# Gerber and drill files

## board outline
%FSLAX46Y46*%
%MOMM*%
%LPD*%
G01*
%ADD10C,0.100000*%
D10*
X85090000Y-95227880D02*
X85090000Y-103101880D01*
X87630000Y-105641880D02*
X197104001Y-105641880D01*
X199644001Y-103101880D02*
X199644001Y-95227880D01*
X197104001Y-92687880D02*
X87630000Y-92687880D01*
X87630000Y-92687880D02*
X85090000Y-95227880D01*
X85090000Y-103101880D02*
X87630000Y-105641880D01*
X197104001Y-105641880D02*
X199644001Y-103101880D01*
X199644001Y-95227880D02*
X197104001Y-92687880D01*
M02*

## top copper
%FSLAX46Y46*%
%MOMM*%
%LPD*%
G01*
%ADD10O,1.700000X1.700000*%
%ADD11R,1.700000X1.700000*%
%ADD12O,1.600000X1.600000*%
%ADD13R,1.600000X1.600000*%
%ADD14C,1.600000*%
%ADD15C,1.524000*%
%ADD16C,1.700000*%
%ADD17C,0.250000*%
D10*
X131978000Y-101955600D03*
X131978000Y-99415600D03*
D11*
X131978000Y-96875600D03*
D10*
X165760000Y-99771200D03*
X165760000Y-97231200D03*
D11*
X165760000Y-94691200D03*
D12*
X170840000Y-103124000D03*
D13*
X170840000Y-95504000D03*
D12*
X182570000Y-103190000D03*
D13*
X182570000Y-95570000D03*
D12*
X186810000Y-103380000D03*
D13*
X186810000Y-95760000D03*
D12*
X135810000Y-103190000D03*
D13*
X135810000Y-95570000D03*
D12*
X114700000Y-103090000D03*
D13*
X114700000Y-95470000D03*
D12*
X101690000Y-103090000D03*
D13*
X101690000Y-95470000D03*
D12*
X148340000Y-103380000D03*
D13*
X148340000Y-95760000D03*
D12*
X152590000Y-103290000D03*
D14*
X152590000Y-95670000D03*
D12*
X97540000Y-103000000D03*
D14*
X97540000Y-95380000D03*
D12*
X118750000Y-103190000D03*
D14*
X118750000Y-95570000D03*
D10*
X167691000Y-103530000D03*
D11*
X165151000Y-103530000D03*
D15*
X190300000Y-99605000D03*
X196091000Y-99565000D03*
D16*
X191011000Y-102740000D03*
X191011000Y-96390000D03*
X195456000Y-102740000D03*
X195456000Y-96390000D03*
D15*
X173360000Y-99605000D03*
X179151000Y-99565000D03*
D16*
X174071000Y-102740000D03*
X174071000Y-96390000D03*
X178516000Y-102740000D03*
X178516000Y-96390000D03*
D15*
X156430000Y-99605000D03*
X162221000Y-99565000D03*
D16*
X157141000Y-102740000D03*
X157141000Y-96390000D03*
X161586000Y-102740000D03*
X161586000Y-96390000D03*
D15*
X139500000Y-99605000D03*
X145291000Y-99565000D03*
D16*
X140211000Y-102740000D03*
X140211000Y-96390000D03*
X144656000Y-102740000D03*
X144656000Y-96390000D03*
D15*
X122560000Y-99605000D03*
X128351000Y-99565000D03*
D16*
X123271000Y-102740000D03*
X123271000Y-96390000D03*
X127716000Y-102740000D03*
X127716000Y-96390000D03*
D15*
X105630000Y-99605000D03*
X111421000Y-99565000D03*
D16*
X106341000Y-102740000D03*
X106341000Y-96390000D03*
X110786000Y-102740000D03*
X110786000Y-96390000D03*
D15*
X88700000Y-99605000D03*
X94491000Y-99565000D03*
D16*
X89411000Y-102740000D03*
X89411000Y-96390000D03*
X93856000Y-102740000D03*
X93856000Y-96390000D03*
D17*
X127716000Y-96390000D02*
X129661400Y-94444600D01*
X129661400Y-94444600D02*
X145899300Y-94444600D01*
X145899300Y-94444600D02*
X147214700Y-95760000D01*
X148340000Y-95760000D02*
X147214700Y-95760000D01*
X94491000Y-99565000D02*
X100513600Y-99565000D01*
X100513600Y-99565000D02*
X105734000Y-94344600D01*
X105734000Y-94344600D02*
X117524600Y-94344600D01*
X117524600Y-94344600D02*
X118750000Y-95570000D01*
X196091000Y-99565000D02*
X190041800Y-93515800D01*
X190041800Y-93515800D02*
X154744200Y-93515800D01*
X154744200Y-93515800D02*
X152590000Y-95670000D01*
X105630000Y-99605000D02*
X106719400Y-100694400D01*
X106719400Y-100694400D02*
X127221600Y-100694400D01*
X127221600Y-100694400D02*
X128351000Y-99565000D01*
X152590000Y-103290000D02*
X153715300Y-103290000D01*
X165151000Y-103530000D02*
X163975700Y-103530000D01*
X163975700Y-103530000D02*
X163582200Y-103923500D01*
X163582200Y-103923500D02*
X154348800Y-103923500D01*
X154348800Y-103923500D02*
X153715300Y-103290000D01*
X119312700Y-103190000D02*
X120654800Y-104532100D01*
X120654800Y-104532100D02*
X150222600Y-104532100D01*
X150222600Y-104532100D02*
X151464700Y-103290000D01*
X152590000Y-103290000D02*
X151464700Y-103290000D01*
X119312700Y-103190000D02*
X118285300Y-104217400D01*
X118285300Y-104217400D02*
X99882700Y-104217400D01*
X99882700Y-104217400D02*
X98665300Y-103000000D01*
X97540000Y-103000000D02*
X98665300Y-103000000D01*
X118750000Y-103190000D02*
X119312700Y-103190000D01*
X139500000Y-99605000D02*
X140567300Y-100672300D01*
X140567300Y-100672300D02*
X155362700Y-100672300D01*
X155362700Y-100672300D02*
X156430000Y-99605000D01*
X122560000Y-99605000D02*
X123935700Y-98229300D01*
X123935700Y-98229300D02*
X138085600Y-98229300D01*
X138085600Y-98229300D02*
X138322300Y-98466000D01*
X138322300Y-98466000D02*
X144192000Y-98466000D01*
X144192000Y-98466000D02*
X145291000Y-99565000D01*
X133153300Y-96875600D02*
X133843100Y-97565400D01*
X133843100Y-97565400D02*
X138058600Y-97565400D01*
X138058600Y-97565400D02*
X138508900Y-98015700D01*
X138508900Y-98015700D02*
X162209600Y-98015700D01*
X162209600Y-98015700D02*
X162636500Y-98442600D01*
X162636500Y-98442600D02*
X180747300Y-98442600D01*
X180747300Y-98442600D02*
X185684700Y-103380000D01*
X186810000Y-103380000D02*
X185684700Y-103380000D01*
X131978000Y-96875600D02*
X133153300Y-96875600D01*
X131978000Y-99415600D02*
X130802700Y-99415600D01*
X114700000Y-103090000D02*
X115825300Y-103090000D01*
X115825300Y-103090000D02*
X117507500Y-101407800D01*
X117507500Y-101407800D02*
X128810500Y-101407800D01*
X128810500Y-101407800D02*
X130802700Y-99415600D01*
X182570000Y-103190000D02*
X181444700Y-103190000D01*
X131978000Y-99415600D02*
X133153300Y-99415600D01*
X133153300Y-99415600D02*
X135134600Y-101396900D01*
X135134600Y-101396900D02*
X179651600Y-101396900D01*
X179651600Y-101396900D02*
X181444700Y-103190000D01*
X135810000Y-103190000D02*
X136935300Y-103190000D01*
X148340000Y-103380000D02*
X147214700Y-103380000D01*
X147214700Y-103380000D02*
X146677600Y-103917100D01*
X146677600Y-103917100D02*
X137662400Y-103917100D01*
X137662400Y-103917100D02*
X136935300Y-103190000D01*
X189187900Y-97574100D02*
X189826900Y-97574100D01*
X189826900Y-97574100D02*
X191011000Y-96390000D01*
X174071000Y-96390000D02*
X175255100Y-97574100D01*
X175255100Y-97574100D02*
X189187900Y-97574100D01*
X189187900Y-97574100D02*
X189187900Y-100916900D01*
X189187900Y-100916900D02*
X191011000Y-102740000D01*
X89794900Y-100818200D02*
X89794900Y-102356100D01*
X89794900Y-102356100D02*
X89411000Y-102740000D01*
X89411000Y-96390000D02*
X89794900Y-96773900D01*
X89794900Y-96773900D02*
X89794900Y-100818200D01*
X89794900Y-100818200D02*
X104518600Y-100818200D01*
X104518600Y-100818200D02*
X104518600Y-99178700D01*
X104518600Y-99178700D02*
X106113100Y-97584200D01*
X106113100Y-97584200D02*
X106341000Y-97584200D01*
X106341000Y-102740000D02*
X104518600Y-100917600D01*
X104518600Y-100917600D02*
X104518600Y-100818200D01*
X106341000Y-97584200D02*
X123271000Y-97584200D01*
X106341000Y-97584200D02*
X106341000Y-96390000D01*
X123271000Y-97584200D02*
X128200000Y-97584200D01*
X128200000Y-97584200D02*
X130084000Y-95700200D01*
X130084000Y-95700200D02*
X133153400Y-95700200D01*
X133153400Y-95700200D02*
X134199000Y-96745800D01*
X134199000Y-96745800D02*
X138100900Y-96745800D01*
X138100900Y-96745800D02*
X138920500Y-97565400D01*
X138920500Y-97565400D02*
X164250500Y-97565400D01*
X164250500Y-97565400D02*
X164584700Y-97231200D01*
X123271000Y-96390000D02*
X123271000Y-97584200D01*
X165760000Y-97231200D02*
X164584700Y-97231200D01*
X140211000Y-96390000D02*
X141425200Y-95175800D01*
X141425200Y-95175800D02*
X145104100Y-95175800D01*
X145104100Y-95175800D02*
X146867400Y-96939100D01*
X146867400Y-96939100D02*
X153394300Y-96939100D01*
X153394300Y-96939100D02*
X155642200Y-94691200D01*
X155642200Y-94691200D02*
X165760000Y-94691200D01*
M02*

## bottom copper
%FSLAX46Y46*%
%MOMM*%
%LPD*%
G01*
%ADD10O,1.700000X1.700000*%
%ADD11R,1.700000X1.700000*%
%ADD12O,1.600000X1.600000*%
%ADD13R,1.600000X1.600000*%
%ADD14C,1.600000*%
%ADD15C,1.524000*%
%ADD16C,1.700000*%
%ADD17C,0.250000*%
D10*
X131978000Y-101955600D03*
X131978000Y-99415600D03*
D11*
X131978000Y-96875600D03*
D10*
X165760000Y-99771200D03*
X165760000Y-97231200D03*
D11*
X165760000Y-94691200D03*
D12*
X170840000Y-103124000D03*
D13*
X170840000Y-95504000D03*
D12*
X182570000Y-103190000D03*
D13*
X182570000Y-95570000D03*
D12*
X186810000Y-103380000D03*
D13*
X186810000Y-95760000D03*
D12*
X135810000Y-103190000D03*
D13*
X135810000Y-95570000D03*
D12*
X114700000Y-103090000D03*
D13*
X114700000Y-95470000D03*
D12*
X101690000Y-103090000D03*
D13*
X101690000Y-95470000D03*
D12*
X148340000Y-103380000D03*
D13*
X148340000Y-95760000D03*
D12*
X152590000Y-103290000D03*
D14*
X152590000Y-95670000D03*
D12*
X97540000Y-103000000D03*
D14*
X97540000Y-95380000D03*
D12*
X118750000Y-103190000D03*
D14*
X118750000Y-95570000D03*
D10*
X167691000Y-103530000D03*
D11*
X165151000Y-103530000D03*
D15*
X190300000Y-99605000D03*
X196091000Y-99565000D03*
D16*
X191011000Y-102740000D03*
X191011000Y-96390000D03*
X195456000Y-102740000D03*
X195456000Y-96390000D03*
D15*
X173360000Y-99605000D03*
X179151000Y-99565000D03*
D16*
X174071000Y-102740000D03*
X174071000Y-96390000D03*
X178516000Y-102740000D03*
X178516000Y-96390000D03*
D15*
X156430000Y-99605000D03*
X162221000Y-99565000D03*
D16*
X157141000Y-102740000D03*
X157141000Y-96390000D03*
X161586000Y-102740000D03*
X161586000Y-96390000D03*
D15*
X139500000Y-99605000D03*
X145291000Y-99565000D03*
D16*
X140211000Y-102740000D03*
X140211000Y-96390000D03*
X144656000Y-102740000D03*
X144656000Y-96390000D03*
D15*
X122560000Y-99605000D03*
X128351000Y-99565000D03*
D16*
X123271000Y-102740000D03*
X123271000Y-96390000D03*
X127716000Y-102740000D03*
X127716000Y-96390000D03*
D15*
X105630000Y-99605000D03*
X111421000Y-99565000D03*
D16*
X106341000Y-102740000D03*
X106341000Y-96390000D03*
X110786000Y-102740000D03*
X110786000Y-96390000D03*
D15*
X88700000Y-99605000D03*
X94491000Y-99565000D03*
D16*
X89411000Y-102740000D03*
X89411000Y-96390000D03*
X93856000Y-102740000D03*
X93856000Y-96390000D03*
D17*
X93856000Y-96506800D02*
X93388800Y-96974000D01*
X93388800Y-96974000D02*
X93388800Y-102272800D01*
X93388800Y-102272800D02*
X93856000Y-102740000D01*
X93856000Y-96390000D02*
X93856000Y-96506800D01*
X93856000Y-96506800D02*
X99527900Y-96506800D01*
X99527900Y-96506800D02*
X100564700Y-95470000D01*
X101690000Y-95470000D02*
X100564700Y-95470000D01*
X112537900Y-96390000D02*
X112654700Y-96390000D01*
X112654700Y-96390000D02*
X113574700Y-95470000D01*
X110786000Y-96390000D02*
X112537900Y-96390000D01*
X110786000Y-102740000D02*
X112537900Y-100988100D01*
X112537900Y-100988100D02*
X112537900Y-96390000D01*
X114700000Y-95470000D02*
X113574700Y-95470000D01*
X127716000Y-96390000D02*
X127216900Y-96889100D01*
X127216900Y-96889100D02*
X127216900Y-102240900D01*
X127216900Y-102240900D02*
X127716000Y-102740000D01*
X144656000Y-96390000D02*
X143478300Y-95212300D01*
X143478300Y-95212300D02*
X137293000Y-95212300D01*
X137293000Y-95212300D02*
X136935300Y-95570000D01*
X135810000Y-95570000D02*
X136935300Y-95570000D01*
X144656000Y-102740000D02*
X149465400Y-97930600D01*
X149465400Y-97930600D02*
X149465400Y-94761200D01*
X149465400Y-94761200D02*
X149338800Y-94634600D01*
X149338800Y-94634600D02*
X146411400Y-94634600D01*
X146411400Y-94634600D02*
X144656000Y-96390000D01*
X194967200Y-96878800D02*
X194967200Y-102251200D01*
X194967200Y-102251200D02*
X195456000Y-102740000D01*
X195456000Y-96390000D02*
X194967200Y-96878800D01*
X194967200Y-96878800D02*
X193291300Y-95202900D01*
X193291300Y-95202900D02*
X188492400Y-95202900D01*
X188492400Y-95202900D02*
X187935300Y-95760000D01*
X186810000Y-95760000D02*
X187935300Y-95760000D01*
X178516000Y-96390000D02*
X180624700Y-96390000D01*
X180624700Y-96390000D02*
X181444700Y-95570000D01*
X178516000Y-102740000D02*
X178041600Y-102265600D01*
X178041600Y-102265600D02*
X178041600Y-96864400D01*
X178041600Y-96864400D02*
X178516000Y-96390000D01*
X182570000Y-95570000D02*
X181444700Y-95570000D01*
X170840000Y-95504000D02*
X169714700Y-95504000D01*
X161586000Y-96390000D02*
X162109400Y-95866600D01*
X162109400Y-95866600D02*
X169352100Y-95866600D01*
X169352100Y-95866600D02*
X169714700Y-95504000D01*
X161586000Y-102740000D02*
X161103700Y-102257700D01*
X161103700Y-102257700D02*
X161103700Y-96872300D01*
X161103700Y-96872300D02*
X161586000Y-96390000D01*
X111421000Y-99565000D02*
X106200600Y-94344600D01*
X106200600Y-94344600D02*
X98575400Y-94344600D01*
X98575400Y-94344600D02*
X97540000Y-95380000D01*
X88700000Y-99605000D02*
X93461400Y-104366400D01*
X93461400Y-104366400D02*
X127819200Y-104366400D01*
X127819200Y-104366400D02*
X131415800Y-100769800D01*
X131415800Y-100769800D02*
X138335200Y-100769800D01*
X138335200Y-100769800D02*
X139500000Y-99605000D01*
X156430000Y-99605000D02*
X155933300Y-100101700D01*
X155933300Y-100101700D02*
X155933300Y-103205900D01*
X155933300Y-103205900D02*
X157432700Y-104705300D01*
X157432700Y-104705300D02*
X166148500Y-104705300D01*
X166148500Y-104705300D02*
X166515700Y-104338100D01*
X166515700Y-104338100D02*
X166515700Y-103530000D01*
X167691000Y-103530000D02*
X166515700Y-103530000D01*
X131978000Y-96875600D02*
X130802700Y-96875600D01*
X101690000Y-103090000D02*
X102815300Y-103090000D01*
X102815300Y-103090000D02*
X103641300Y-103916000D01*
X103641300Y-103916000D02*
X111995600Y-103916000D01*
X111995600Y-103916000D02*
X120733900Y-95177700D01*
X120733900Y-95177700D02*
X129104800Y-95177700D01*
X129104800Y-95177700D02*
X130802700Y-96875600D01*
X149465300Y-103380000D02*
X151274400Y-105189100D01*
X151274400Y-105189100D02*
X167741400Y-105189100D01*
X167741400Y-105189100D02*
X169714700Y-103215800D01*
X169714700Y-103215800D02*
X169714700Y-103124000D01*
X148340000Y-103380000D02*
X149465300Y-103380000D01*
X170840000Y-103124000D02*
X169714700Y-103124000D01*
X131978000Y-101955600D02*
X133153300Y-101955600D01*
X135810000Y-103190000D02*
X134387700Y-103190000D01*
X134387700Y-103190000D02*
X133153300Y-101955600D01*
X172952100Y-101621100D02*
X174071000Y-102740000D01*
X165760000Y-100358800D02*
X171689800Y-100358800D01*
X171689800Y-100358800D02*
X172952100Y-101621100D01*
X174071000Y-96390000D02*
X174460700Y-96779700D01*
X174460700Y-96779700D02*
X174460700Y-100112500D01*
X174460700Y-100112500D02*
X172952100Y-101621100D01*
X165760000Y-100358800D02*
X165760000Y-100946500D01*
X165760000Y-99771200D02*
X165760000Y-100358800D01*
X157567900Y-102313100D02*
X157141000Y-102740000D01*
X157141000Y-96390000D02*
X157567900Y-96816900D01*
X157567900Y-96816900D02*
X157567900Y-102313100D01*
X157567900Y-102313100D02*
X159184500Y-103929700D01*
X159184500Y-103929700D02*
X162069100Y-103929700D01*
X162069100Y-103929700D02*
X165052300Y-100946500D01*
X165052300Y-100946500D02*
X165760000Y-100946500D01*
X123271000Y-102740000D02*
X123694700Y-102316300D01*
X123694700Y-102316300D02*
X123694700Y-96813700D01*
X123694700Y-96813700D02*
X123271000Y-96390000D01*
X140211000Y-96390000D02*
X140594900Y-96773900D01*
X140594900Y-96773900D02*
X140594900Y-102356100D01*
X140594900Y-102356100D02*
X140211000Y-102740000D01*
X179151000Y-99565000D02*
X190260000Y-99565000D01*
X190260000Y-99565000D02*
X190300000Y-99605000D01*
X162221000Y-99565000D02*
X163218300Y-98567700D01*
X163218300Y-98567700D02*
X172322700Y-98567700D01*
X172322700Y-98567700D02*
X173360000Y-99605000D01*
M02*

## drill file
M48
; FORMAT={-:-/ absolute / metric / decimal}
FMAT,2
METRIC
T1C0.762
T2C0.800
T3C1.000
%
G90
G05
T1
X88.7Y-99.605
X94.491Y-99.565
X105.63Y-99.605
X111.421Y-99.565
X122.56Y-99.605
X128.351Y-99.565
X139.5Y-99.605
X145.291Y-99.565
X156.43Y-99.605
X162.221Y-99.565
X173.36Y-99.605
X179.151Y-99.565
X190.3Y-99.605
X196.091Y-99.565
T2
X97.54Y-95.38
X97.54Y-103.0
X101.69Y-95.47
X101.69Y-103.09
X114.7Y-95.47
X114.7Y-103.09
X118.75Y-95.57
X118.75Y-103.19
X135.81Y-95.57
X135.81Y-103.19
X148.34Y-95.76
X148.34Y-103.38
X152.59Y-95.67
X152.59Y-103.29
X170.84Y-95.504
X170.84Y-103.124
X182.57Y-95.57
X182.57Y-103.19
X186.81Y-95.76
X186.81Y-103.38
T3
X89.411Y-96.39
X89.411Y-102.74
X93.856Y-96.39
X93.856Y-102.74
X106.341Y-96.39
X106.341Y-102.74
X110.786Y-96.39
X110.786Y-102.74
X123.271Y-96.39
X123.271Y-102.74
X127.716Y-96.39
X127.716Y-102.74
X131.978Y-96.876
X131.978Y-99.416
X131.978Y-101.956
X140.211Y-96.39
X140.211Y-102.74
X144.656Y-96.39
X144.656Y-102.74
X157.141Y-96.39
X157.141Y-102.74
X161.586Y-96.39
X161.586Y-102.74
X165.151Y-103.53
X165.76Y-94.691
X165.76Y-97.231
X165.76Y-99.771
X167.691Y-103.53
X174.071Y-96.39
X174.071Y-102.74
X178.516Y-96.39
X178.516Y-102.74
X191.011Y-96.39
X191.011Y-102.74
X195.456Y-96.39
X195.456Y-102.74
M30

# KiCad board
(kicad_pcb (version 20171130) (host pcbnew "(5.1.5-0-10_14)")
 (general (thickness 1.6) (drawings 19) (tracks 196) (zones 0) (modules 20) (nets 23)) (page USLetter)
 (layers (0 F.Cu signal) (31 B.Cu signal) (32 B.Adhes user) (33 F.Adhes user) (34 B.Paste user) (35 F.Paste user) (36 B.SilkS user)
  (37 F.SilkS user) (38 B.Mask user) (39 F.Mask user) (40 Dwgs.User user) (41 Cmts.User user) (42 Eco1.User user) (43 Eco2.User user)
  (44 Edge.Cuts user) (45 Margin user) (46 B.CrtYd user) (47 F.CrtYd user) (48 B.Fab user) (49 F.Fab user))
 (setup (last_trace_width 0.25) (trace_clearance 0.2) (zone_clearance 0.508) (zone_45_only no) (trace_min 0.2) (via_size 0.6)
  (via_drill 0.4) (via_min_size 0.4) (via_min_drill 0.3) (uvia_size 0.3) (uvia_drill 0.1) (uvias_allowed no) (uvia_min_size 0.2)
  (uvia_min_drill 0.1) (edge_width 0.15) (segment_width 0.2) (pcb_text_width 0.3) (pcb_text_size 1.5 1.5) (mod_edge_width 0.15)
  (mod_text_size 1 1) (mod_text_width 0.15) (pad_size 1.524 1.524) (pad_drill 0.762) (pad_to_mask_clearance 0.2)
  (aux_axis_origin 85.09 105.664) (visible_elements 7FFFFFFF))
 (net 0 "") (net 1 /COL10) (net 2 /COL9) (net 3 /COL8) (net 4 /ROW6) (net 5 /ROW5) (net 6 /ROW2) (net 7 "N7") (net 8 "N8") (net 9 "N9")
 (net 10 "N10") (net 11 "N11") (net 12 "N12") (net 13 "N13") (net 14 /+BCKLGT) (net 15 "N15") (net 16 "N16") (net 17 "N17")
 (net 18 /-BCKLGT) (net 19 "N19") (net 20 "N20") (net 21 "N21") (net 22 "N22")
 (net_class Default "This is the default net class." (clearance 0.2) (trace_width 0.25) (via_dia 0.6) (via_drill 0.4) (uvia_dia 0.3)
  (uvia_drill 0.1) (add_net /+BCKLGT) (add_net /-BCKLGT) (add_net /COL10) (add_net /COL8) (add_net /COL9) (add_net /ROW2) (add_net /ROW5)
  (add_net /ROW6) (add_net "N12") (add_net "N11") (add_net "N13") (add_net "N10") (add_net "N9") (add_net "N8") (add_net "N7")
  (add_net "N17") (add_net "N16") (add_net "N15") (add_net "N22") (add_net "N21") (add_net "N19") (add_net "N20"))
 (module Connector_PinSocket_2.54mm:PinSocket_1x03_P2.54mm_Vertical (layer F.Cu) (at 131.978 96.8756)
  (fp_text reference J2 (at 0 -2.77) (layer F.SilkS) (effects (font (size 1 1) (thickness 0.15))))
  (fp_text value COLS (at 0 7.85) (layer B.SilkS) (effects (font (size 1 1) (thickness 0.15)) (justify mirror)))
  (pad 3 thru_hole oval (at 0 5.08) (size 1.7 1.7) (drill 1) (layers *.Cu *.Mask) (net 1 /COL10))
  (pad 2 thru_hole oval (at 0 2.54) (size 1.7 1.7) (drill 1) (layers *.Cu *.Mask) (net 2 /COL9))
  (pad 1 thru_hole rect (at 0 0) (size 1.7 1.7) (drill 1) (layers *.Cu *.Mask) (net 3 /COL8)))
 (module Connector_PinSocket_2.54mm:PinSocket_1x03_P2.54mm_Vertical (layer F.Cu) (at 165.76 94.6912)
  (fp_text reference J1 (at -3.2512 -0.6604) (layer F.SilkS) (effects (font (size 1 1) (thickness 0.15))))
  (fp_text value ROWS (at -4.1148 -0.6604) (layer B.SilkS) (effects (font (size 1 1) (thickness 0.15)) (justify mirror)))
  (pad 3 thru_hole oval (at 0 5.08) (size 1.7 1.7) (drill 1) (layers *.Cu *.Mask) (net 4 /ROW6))
  (pad 2 thru_hole oval (at 0 2.54) (size 1.7 1.7) (drill 1) (layers *.Cu *.Mask) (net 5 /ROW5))
  (pad 1 thru_hole rect (at 0 0) (size 1.7 1.7) (drill 1) (layers *.Cu *.Mask) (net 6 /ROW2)))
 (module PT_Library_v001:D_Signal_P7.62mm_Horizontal (layer F.Cu) (at 170.84 95.504 270)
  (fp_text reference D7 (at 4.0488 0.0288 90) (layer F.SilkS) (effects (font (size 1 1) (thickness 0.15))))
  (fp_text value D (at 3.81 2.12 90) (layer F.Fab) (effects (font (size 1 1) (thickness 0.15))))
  (pad 2 thru_hole oval (at 7.62 0 270) (size 1.6 1.6) (drill 0.8) (layers *.Cu *.Mask) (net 1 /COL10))
  (pad 1 thru_hole rect (at 0 0 270) (size 1.6 1.6) (drill 0.8) (layers *.Cu *.Mask) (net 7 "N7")))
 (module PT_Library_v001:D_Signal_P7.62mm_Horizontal (layer F.Cu) (at 182.57 95.57 270)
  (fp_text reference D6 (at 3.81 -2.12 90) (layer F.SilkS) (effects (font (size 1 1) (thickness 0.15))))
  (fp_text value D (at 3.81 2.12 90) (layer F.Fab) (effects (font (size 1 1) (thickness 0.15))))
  (pad 2 thru_hole oval (at 7.62 0 270) (size 1.6 1.6) (drill 0.8) (layers *.Cu *.Mask) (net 2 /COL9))
  (pad 1 thru_hole rect (at 0 0 270) (size 1.6 1.6) (drill 0.8) (layers *.Cu *.Mask) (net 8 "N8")))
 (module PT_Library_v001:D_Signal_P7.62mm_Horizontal (layer F.Cu) (at 186.81 95.76 270)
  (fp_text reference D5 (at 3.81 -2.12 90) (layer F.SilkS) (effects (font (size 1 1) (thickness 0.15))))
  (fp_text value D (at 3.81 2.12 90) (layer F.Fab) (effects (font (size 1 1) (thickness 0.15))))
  (pad 2 thru_hole oval (at 7.62 0 270) (size 1.6 1.6) (drill 0.8) (layers *.Cu *.Mask) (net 3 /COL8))
  (pad 1 thru_hole rect (at 0 0 270) (size 1.6 1.6) (drill 0.8) (layers *.Cu *.Mask) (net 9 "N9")))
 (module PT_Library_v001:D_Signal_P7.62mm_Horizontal (layer F.Cu) (at 135.81 95.57 270)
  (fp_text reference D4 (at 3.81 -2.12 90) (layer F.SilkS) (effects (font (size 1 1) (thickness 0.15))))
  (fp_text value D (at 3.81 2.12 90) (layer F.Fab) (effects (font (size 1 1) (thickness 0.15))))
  (pad 2 thru_hole oval (at 7.62 0 270) (size 1.6 1.6) (drill 0.8) (layers *.Cu *.Mask) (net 1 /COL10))
  (pad 1 thru_hole rect (at 0 0 270) (size 1.6 1.6) (drill 0.8) (layers *.Cu *.Mask) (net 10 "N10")))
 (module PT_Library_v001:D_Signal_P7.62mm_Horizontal (layer F.Cu) (at 114.7 95.47 270)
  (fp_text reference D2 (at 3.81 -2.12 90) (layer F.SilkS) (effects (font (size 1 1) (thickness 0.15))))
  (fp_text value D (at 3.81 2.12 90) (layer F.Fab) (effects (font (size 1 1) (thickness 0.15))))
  (pad 2 thru_hole oval (at 7.62 0 270) (size 1.6 1.6) (drill 0.8) (layers *.Cu *.Mask) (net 2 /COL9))
  (pad 1 thru_hole rect (at 0 0 270) (size 1.6 1.6) (drill 0.8) (layers *.Cu *.Mask) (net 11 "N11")))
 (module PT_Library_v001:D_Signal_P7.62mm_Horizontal (layer F.Cu) (at 101.69 95.47 270)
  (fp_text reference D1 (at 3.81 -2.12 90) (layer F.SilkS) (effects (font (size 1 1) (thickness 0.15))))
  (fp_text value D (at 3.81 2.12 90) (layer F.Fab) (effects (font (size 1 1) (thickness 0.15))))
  (pad 2 thru_hole oval (at 7.62 0 270) (size 1.6 1.6) (drill 0.8) (layers *.Cu *.Mask) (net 3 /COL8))
  (pad 1 thru_hole rect (at 0 0 270) (size 1.6 1.6) (drill 0.8) (layers *.Cu *.Mask) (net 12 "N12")))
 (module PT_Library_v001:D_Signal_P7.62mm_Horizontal (layer F.Cu) (at 148.34 95.76 270)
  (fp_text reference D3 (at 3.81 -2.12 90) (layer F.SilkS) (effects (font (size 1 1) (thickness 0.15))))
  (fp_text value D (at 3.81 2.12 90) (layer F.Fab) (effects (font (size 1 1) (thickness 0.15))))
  (pad 2 thru_hole oval (at 7.62 0 270) (size 1.6 1.6) (drill 0.8) (layers *.Cu *.Mask) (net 1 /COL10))
  (pad 1 thru_hole rect (at 0 0 270) (size 1.6 1.6) (drill 0.8) (layers *.Cu *.Mask) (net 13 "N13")))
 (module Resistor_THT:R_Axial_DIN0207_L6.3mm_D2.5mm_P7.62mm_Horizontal (layer F.Cu) (at 152.59 95.67 270)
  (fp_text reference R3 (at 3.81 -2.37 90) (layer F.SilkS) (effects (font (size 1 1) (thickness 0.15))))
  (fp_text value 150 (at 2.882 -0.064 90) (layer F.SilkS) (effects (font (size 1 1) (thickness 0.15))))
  (pad 2 thru_hole oval (at 7.62 0 270) (size 1.6 1.6) (drill 0.8) (layers *.Cu *.Mask) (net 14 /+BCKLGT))
  (pad 1 thru_hole circle (at 0 0 270) (size 1.6 1.6) (drill 0.8) (layers *.Cu *.Mask) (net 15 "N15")))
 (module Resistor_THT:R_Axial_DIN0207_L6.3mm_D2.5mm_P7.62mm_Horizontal (layer F.Cu) (at 97.54 95.38 270)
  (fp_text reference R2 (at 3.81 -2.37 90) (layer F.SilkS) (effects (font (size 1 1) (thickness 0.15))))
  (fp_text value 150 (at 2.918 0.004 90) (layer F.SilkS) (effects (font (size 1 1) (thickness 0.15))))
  (pad 2 thru_hole oval (at 7.62 0 270) (size 1.6 1.6) (drill 0.8) (layers *.Cu *.Mask) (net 14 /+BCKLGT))
  (pad 1 thru_hole circle (at 0 0 270) (size 1.6 1.6) (drill 0.8) (layers *.Cu *.Mask) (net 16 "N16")))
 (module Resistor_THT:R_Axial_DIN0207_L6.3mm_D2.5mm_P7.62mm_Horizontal (layer F.Cu) (at 118.75 95.57 270)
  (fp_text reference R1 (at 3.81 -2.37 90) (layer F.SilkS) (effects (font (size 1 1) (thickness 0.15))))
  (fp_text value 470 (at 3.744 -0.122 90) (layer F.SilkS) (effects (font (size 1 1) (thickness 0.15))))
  (pad 2 thru_hole oval (at 7.62 0 270) (size 1.6 1.6) (drill 0.8) (layers *.Cu *.Mask) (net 14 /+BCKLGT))
  (pad 1 thru_hole circle (at 0 0 270) (size 1.6 1.6) (drill 0.8) (layers *.Cu *.Mask) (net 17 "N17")))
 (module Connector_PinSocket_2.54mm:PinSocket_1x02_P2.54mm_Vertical (layer B.Cu) (at 165.151 103.53 270)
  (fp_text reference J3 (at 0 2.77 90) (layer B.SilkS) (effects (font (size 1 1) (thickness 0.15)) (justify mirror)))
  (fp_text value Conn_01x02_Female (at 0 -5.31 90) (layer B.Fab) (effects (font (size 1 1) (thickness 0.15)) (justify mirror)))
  (pad 2 thru_hole oval (at 0 -2.54 270) (size 1.7 1.7) (drill 1) (layers *.Cu *.Mask) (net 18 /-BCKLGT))
  (pad 1 thru_hole rect (at 0 0 270) (size 1.7 1.7) (drill 1) (layers *.Cu *.Mask) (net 14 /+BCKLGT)))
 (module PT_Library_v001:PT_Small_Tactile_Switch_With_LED (layer F.Cu) (at 193.17 99.565 270)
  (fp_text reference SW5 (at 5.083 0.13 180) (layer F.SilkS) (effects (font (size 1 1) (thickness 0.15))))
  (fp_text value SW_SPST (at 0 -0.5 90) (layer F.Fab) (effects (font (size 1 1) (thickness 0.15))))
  (pad 6 thru_hole circle (at 0.04 2.87 270) (size 1.524 1.524) (drill 0.762) (layers *.Cu *.Mask) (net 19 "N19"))
  (pad 5 thru_hole circle (at 0 -2.921 270) (size 1.524 1.524) (drill 0.762) (layers *.Cu *.Mask) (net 15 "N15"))
  (pad 4 thru_hole circle (at 3.175 2.159 270) (size 1.7 1.7) (drill 1) (layers *.Cu *.Mask) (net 4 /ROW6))
  (pad 3 thru_hole circle (at -3.175 2.159 270) (size 1.7 1.7) (drill 1) (layers *.Cu *.Mask) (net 4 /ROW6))
  (pad 2 thru_hole circle (at 3.175 -2.286 270) (size 1.7 1.7) (drill 1) (layers *.Cu *.Mask) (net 9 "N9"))
  (pad 1 thru_hole circle (at -3.175 -2.286 270) (size 1.7 1.7) (drill 1) (layers *.Cu *.Mask) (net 9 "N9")))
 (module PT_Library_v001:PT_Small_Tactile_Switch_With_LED (layer F.Cu) (at 176.23 99.565 270)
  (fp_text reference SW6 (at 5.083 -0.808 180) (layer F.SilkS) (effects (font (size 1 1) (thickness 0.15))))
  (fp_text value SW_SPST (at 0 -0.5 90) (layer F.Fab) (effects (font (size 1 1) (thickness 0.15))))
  (pad 6 thru_hole circle (at 0.04 2.87 270) (size 1.524 1.524) (drill 0.762) (layers *.Cu *.Mask) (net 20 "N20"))
  (pad 5 thru_hole circle (at 0 -2.921 270) (size 1.524 1.524) (drill 0.762) (layers *.Cu *.Mask) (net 19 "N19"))
  (pad 4 thru_hole circle (at 3.175 2.159 270) (size 1.7 1.7) (drill 1) (layers *.Cu *.Mask) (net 4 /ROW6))
  (pad 3 thru_hole circle (at -3.175 2.159 270) (size 1.7 1.7) (drill 1) (layers *.Cu *.Mask) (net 4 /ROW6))
  (pad 2 thru_hole circle (at 3.175 -2.286 270) (size 1.7 1.7) (drill 1) (layers *.Cu *.Mask) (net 8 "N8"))
  (pad 1 thru_hole circle (at -3.175 -2.286 270) (size 1.7 1.7) (drill 1) (layers *.Cu *.Mask) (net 8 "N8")))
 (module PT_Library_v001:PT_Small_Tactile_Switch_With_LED (layer F.Cu) (at 159.3 99.565 270)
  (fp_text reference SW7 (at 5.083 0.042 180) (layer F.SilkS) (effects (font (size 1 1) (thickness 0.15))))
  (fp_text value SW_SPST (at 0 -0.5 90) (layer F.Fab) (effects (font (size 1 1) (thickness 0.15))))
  (pad 6 thru_hole circle (at 0.04 2.87 270) (size 1.524 1.524) (drill 0.762) (layers *.Cu *.Mask) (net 18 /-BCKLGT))
  (pad 5 thru_hole circle (at 0 -2.921 270) (size 1.524 1.524) (drill 0.762) (layers *.Cu *.Mask) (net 20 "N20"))
  (pad 4 thru_hole circle (at 3.175 2.159 270) (size 1.7 1.7) (drill 1) (layers *.Cu *.Mask) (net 4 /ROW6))
  (pad 3 thru_hole circle (at -3.175 2.159 270) (size 1.7 1.7) (drill 1) (layers *.Cu *.Mask) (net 4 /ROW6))
  (pad 2 thru_hole circle (at 3.175 -2.286 270) (size 1.7 1.7) (drill 1) (layers *.Cu *.Mask) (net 7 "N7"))
  (pad 1 thru_hole circle (at -3.175 -2.286 270) (size 1.7 1.7) (drill 1) (layers *.Cu *.Mask) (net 7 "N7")))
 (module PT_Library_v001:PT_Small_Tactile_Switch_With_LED (layer F.Cu) (at 142.37 99.565 270)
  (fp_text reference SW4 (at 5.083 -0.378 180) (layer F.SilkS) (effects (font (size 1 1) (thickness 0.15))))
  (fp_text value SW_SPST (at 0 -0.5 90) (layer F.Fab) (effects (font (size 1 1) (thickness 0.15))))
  (pad 6 thru_hole circle (at 0.04 2.87 270) (size 1.524 1.524) (drill 0.762) (layers *.Cu *.Mask) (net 18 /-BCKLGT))
  (pad 5 thru_hole circle (at 0 -2.921 270) (size 1.524 1.524) (drill 0.762) (layers *.Cu *.Mask) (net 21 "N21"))
  (pad 4 thru_hole circle (at 3.175 2.159 270) (size 1.7 1.7) (drill 1) (layers *.Cu *.Mask) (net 6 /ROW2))
  (pad 3 thru_hole circle (at -3.175 2.159 270) (size 1.7 1.7) (drill 1) (layers *.Cu *.Mask) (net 6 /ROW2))
  (pad 2 thru_hole circle (at 3.175 -2.286 270) (size 1.7 1.7) (drill 1) (layers *.Cu *.Mask) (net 10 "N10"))
  (pad 1 thru_hole circle (at -3.175 -2.286 270) (size 1.7 1.7) (drill 1) (layers *.Cu *.Mask) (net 10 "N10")))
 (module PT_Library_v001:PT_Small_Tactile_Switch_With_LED (layer F.Cu) (at 125.43 99.565 270)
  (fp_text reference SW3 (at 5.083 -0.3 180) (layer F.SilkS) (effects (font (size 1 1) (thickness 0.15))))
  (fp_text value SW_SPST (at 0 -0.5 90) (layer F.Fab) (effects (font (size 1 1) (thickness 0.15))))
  (pad 6 thru_hole circle (at 0.04 2.87 270) (size 1.524 1.524) (drill 0.762) (layers *.Cu *.Mask) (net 21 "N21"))
  (pad 5 thru_hole circle (at 0 -2.921 270) (size 1.524 1.524) (drill 0.762) (layers *.Cu *.Mask) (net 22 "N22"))
  (pad 4 thru_hole circle (at 3.175 2.159 270) (size 1.7 1.7) (drill 1) (layers *.Cu *.Mask) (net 5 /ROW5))
  (pad 3 thru_hole circle (at -3.175 2.159 270) (size 1.7 1.7) (drill 1) (layers *.Cu *.Mask) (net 5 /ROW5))
  (pad 2 thru_hole circle (at 3.175 -2.286 270) (size 1.7 1.7) (drill 1) (layers *.Cu *.Mask) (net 13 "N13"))
  (pad 1 thru_hole circle (at -3.175 -2.286 270) (size 1.7 1.7) (drill 1) (layers *.Cu *.Mask) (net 13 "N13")))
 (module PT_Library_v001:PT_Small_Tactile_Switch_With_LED (layer F.Cu) (at 108.5 99.565 270)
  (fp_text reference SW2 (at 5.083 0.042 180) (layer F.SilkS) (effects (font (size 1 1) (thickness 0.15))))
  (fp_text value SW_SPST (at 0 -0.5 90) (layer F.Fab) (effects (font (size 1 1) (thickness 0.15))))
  (pad 6 thru_hole circle (at 0.04 2.87 270) (size 1.524 1.524) (drill 0.762) (layers *.Cu *.Mask) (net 22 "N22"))
  (pad 5 thru_hole circle (at 0 -2.921 270) (size 1.524 1.524) (drill 0.762) (layers *.Cu *.Mask) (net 16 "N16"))
  (pad 4 thru_hole circle (at 3.175 2.159 270) (size 1.7 1.7) (drill 1) (layers *.Cu *.Mask) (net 5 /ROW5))
  (pad 3 thru_hole circle (at -3.175 2.159 270) (size 1.7 1.7) (drill 1) (layers *.Cu *.Mask) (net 5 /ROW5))
  (pad 2 thru_hole circle (at 3.175 -2.286 270) (size 1.7 1.7) (drill 1) (layers *.Cu *.Mask) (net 11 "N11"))
  (pad 1 thru_hole circle (at -3.175 -2.286 270) (size 1.7 1.7) (drill 1) (layers *.Cu *.Mask) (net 11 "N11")))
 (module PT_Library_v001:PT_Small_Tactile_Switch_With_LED (layer F.Cu) (at 91.57 99.565 270)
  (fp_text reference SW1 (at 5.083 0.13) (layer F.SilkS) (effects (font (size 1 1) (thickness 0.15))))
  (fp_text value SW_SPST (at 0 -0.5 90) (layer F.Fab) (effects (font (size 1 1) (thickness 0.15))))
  (pad 6 thru_hole circle (at 0.04 2.87 270) (size 1.524 1.524) (drill 0.762) (layers *.Cu *.Mask) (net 18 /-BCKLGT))
  (pad 5 thru_hole circle (at 0 -2.921 270) (size 1.524 1.524) (drill 0.762) (layers *.Cu *.Mask) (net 17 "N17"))
  (pad 4 thru_hole circle (at 3.175 2.159 270) (size 1.7 1.7) (drill 1) (layers *.Cu *.Mask) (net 5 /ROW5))
  (pad 3 thru_hole circle (at -3.175 2.159 270) (size 1.7 1.7) (drill 1) (layers *.Cu *.Mask) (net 5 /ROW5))
  (pad 2 thru_hole circle (at 3.175 -2.286 270) (size 1.7 1.7) (drill 1) (layers *.Cu *.Mask) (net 12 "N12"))
  (pad 1 thru_hole circle (at -3.175 -2.286 270) (size 1.7 1.7) (drill 1) (layers *.Cu *.Mask) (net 12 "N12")))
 (gr_line (start 85.09 95.22788) (end 85.09 103.10188) (layer Edge.Cuts) (width 0.1))
 (gr_line (start 87.63 105.64188) (end 197.104001 105.64188) (layer Edge.Cuts) (width 0.1))
 (gr_line (start 199.644001 103.10188) (end 199.644001 95.22788) (layer Edge.Cuts) (width 0.1))
 (gr_line (start 197.104001 92.68788) (end 87.63 92.68788) (layer Edge.Cuts) (width 0.1))
 (gr_line (start 87.63 92.68788) (end 85.09 95.22788) (layer Edge.Cuts) (width 0.1))
 (gr_line (start 85.09 103.10188) (end 87.63 105.64188) (layer Edge.Cuts) (width 0.1))
 (gr_line (start 197.104001 105.64188) (end 199.644001 103.10188) (layer Edge.Cuts) (width 0.1))
 (gr_line (start 199.644001 95.22788) (end 197.104001 92.68788) (layer Edge.Cuts) (width 0.1))
 (segment (start 93.856 96.5068) (end 93.3888 96.974) (width 0.25) (layer B.Cu) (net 12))
 (segment (start 93.3888 96.974) (end 93.3888 102.2728) (width 0.25) (layer B.Cu) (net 12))
 (segment (start 93.3888 102.2728) (end 93.856 102.74) (width 0.25) (layer B.Cu) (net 12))
 (segment (start 93.856 96.39) (end 93.856 96.5068) (width 0.25) (layer B.Cu) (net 12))
 (segment (start 93.856 96.5068) (end 99.5279 96.5068) (width 0.25) (layer B.Cu) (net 12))
 (segment (start 99.5279 96.5068) (end 100.5647 95.47) (width 0.25) (layer B.Cu) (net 12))
 (segment (start 101.69 95.47) (end 100.5647 95.47) (width 0.25) (layer B.Cu) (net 12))
 (segment (start 112.5379 96.39) (end 112.6547 96.39) (width 0.25) (layer B.Cu) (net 11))
 (segment (start 112.6547 96.39) (end 113.5747 95.47) (width 0.25) (layer B.Cu) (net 11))
 (segment (start 110.786 96.39) (end 112.5379 96.39) (width 0.25) (layer B.Cu) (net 11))
 (segment (start 110.786 102.74) (end 112.5379 100.9881) (width 0.25) (layer B.Cu) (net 11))
 (segment (start 112.5379 100.9881) (end 112.5379 96.39) (width 0.25) (layer B.Cu) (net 11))
 (segment (start 114.7 95.47) (end 113.5747 95.47) (width 0.25) (layer B.Cu) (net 11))
 (segment (start 127.716 96.39) (end 127.2169 96.8891) (width 0.25) (layer B.Cu) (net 13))
 (segment (start 127.2169 96.8891) (end 127.2169 102.2409) (width 0.25) (layer B.Cu) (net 13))
 (segment (start 127.2169 102.2409) (end 127.716 102.74) (width 0.25) (layer B.Cu) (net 13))
 (segment (start 127.716 96.39) (end 129.6614 94.4446) (width 0.25) (layer F.Cu) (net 13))
 (segment (start 129.6614 94.4446) (end 145.8993 94.4446) (width 0.25) (layer F.Cu) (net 13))
 (segment (start 145.8993 94.4446) (end 147.2147 95.76) (width 0.25) (layer F.Cu) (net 13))
 (segment (start 148.34 95.76) (end 147.2147 95.76) (width 0.25) (layer F.Cu) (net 13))
 (segment (start 144.656 96.39) (end 143.4783 95.2123) (width 0.25) (layer B.Cu) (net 10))
 (segment (start 143.4783 95.2123) (end 137.293 95.2123) (width 0.25) (layer B.Cu) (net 10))
 (segment (start 137.293 95.2123) (end 136.9353 95.57) (width 0.25) (layer B.Cu) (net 10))
 (segment (start 135.81 95.57) (end 136.9353 95.57) (width 0.25) (layer B.Cu) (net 10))
 (segment (start 144.656 102.74) (end 149.4654 97.9306) (width 0.25) (layer B.Cu) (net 10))
 (segment (start 149.4654 97.9306) (end 149.4654 94.7612) (width 0.25) (layer B.Cu) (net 10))
 (segment (start 149.4654 94.7612) (end 149.3388 94.6346) (width 0.25) (layer B.Cu) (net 10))
 (segment (start 149.3388 94.6346) (end 146.4114 94.6346) (width 0.25) (layer B.Cu) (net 10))
 (segment (start 146.4114 94.6346) (end 144.656 96.39) (width 0.25) (layer B.Cu) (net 10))
 (segment (start 194.9672 96.8788) (end 194.9672 102.2512) (width 0.25) (layer B.Cu) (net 9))
 (segment (start 194.9672 102.2512) (end 195.456 102.74) (width 0.25) (layer B.Cu) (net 9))
 (segment (start 195.456 96.39) (end 194.9672 96.8788) (width 0.25) (layer B.Cu) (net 9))
 (segment (start 194.9672 96.8788) (end 193.2913 95.2029) (width 0.25) (layer B.Cu) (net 9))
 (segment (start 193.2913 95.2029) (end 188.4924 95.2029) (width 0.25) (layer B.Cu) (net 9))
 (segment (start 188.4924 95.2029) (end 187.9353 95.76) (width 0.25) (layer B.Cu) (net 9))
 (segment (start 186.81 95.76) (end 187.9353 95.76) (width 0.25) (layer B.Cu) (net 9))
 (segment (start 178.516 96.39) (end 180.6247 96.39) (width 0.25) (layer B.Cu) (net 8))
 (segment (start 180.6247 96.39) (end 181.4447 95.57) (width 0.25) (layer B.Cu) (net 8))
 (segment (start 178.516 102.74) (end 178.0416 102.2656) (width 0.25) (layer B.Cu) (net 8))
 (segment (start 178.0416 102.2656) (end 178.0416 96.8644) (width 0.25) (layer B.Cu) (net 8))
 (segment (start 178.0416 96.8644) (end 178.516 96.39) (width 0.25) (layer B.Cu) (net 8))
 (segment (start 182.57 95.57) (end 181.4447 95.57) (width 0.25) (layer B.Cu) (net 8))
 (segment (start 170.84 95.504) (end 169.7147 95.504) (width 0.25) (layer B.Cu) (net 7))
 (segment (start 161.586 96.39) (end 162.1094 95.8666) (width 0.25) (layer B.Cu) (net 7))
 (segment (start 162.1094 95.8666) (end 169.3521 95.8666) (width 0.25) (layer B.Cu) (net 7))
 (segment (start 169.3521 95.8666) (end 169.7147 95.504) (width 0.25) (layer B.Cu) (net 7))
 (segment (start 161.586 102.74) (end 161.1037 102.2577) (width 0.25) (layer B.Cu) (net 7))
 (segment (start 161.1037 102.2577) (end 161.1037 96.8723) (width 0.25) (layer B.Cu) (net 7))
 (segment (start 161.1037 96.8723) (end 161.586 96.39) (width 0.25) (layer B.Cu) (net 7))
 (segment (start 94.491 99.565) (end 100.5136 99.565) (width 0.25) (layer F.Cu) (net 17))
 (segment (start 100.5136 99.565) (end 105.734 94.3446) (width 0.25) (layer F.Cu) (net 17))
 (segment (start 105.734 94.3446) (end 117.5246 94.3446) (width 0.25) (layer F.Cu) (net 17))
 (segment (start 117.5246 94.3446) (end 118.75 95.57) (width 0.25) (layer F.Cu) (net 17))
 (segment (start 111.421 99.565) (end 106.2006 94.3446) (width 0.25) (layer B.Cu) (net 16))
 (segment (start 106.2006 94.3446) (end 98.5754 94.3446) (width 0.25) (layer B.Cu) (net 16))
 (segment (start 98.5754 94.3446) (end 97.54 95.38) (width 0.25) (layer B.Cu) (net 16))
 (segment (start 196.091 99.565) (end 190.0418 93.5158) (width 0.25) (layer F.Cu) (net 15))
 (segment (start 190.0418 93.5158) (end 154.7442 93.5158) (width 0.25) (layer F.Cu) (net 15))
 (segment (start 154.7442 93.5158) (end 152.59 95.67) (width 0.25) (layer F.Cu) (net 15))
 (segment (start 105.63 99.605) (end 106.7194 100.6944) (width 0.25) (layer F.Cu) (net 22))
 (segment (start 106.7194 100.6944) (end 127.2216 100.6944) (width 0.25) (layer F.Cu) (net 22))
 (segment (start 127.2216 100.6944) (end 128.351 99.565) (width 0.25) (layer F.Cu) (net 22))
 (segment (start 152.59 103.29) (end 153.7153 103.29) (width 0.25) (layer F.Cu) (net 14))
 (segment (start 165.151 103.53) (end 163.9757 103.53) (width 0.25) (layer F.Cu) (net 14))
 (segment (start 163.9757 103.53) (end 163.5822 103.9235) (width 0.25) (layer F.Cu) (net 14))
 (segment (start 163.5822 103.9235) (end 154.3488 103.9235) (width 0.25) (layer F.Cu) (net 14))
 (segment (start 154.3488 103.9235) (end 153.7153 103.29) (width 0.25) (layer F.Cu) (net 14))
 (segment (start 119.3127 103.19) (end 120.6548 104.5321) (width 0.25) (layer F.Cu) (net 14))
 (segment (start 120.6548 104.5321) (end 150.2226 104.5321) (width 0.25) (layer F.Cu) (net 14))
 (segment (start 150.2226 104.5321) (end 151.4647 103.29) (width 0.25) (layer F.Cu) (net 14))
 (segment (start 152.59 103.29) (end 151.4647 103.29) (width 0.25) (layer F.Cu) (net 14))
 (segment (start 119.3127 103.19) (end 118.2853 104.2174) (width 0.25) (layer F.Cu) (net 14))
 (segment (start 118.2853 104.2174) (end 99.8827 104.2174) (width 0.25) (layer F.Cu) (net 14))
 (segment (start 99.8827 104.2174) (end 98.6653 103) (width 0.25) (layer F.Cu) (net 14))
 (segment (start 97.54 103) (end 98.6653 103) (width 0.25) (layer F.Cu) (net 14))
 (segment (start 118.75 103.19) (end 119.3127 103.19) (width 0.25) (layer F.Cu) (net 14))
 (segment (start 88.7 99.605) (end 93.4614 104.3664) (width 0.25) (layer B.Cu) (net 18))
 (segment (start 93.4614 104.3664) (end 127.8192 104.3664) (width 0.25) (layer B.Cu) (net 18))
 (segment (start 127.8192 104.3664) (end 131.4158 100.7698) (width 0.25) (layer B.Cu) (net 18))
 (segment (start 131.4158 100.7698) (end 138.3352 100.7698) (width 0.25) (layer B.Cu) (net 18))
 (segment (start 138.3352 100.7698) (end 139.5 99.605) (width 0.25) (layer B.Cu) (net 18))
 (segment (start 139.5 99.605) (end 140.5673 100.6723) (width 0.25) (layer F.Cu) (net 18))
 (segment (start 140.5673 100.6723) (end 155.3627 100.6723) (width 0.25) (layer F.Cu) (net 18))
 (segment (start 155.3627 100.6723) (end 156.43 99.605) (width 0.25) (layer F.Cu) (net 18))
 (segment (start 156.43 99.605) (end 155.9333 100.1017) (width 0.25) (layer B.Cu) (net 18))
 (segment (start 155.9333 100.1017) (end 155.9333 103.2059) (width 0.25) (layer B.Cu) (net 18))
 (segment (start 155.9333 103.2059) (end 157.4327 104.7053) (width 0.25) (layer B.Cu) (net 18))
 (segment (start 157.4327 104.7053) (end 166.1485 104.7053) (width 0.25) (layer B.Cu) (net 18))
 (segment (start 166.1485 104.7053) (end 166.5157 104.3381) (width 0.25) (layer B.Cu) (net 18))
 (segment (start 166.5157 104.3381) (end 166.5157 103.53) (width 0.25) (layer B.Cu) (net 18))
 (segment (start 167.691 103.53) (end 166.5157 103.53) (width 0.25) (layer B.Cu) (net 18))
 (segment (start 122.56 99.605) (end 123.9357 98.2293) (width 0.25) (layer F.Cu) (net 21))
 (segment (start 123.9357 98.2293) (end 138.0856 98.2293) (width 0.25) (layer F.Cu) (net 21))
 (segment (start 138.0856 98.2293) (end 138.3223 98.466) (width 0.25) (layer F.Cu) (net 21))
 (segment (start 138.3223 98.466) (end 144.192 98.466) (width 0.25) (layer F.Cu) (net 21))
 (segment (start 144.192 98.466) (end 145.291 99.565) (width 0.25) (layer F.Cu) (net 21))
 (segment (start 133.1533 96.8756) (end 133.8431 97.5654) (width 0.25) (layer F.Cu) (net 3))
 (segment (start 133.8431 97.5654) (end 138.0586 97.5654) (width 0.25) (layer F.Cu) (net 3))
 (segment (start 138.0586 97.5654) (end 138.5089 98.0157) (width 0.25) (layer F.Cu) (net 3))
 (segment (start 138.5089 98.0157) (end 162.2096 98.0157) (width 0.25) (layer F.Cu) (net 3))
 (segment (start 162.2096 98.0157) (end 162.6365 98.4426) (width 0.25) (layer F.Cu) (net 3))
 (segment (start 162.6365 98.4426) (end 180.7473 98.4426) (width 0.25) (layer F.Cu) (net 3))
 (segment (start 180.7473 98.4426) (end 185.6847 103.38) (width 0.25) (layer F.Cu) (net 3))
 (segment (start 131.978 96.8756) (end 130.8027 96.8756) (width 0.25) (layer B.Cu) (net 3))
 (segment (start 101.69 103.09) (end 102.8153 103.09) (width 0.25) (layer B.Cu) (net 3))
 (segment (start 102.8153 103.09) (end 103.6413 103.916) (width 0.25) (layer B.Cu) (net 3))
 (segment (start 103.6413 103.916) (end 111.9956 103.916) (width 0.25) (layer B.Cu) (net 3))
 (segment (start 111.9956 103.916) (end 120.7339 95.1777) (width 0.25) (layer B.Cu) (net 3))
 (segment (start 120.7339 95.1777) (end 129.1048 95.1777) (width 0.25) (layer B.Cu) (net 3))
 (segment (start 129.1048 95.1777) (end 130.8027 96.8756) (width 0.25) (layer B.Cu) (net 3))
 (segment (start 186.81 103.38) (end 185.6847 103.38) (width 0.25) (layer F.Cu) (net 3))
 (segment (start 131.978 96.8756) (end 133.1533 96.8756) (width 0.25) (layer F.Cu) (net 3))
 (segment (start 131.978 99.4156) (end 130.8027 99.4156) (width 0.25) (layer F.Cu) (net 2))
 (segment (start 114.7 103.09) (end 115.8253 103.09) (width 0.25) (layer F.Cu) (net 2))
 (segment (start 115.8253 103.09) (end 117.5075 101.4078) (width 0.25) (layer F.Cu) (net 2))
 (segment (start 117.5075 101.4078) (end 128.8105 101.4078) (width 0.25) (layer F.Cu) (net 2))
 (segment (start 128.8105 101.4078) (end 130.8027 99.4156) (width 0.25) (layer F.Cu) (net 2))
 (segment (start 182.57 103.19) (end 181.4447 103.19) (width 0.25) (layer F.Cu) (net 2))
 (segment (start 131.978 99.4156) (end 133.1533 99.4156) (width 0.25) (layer F.Cu) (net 2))
 (segment (start 133.1533 99.4156) (end 135.1346 101.3969) (width 0.25) (layer F.Cu) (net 2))
 (segment (start 135.1346 101.3969) (end 179.6516 101.3969) (width 0.25) (layer F.Cu) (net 2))
 (segment (start 179.6516 101.3969) (end 181.4447 103.19) (width 0.25) (layer F.Cu) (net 2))
 (segment (start 135.81 103.19) (end 136.9353 103.19) (width 0.25) (layer F.Cu) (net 1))
 (segment (start 148.34 103.38) (end 147.2147 103.38) (width 0.25) (layer F.Cu) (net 1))
 (segment (start 147.2147 103.38) (end 146.6776 103.9171) (width 0.25) (layer F.Cu) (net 1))
 (segment (start 146.6776 103.9171) (end 137.6624 103.9171) (width 0.25) (layer F.Cu) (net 1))
 (segment (start 137.6624 103.9171) (end 136.9353 103.19) (width 0.25) (layer F.Cu) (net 1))
 (segment (start 149.4653 103.38) (end 151.2744 105.1891) (width 0.25) (layer B.Cu) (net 1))
 (segment (start 151.2744 105.1891) (end 167.7414 105.1891) (width 0.25) (layer B.Cu) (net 1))
 (segment (start 167.7414 105.1891) (end 169.7147 103.2158) (width 0.25) (layer B.Cu) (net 1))
 (segment (start 169.7147 103.2158) (end 169.7147 103.124) (width 0.25) (layer B.Cu) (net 1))
 (segment (start 148.34 103.38) (end 149.4653 103.38) (width 0.25) (layer B.Cu) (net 1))
 (segment (start 170.84 103.124) (end 169.7147 103.124) (width 0.25) (layer B.Cu) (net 1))
 (segment (start 131.978 101.9556) (end 133.1533 101.9556) (width 0.25) (layer B.Cu) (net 1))
 (segment (start 135.81 103.19) (end 134.3877 103.19) (width 0.25) (layer B.Cu) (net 1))
 (segment (start 134.3877 103.19) (end 133.1533 101.9556) (width 0.25) (layer B.Cu) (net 1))
 (segment (start 189.1879 97.5741) (end 189.8269 97.5741) (width 0.25) (layer F.Cu) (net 4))
 (segment (start 189.8269 97.5741) (end 191.011 96.39) (width 0.25) (layer F.Cu) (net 4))
 (segment (start 174.071 96.39) (end 175.2551 97.5741) (width 0.25) (layer F.Cu) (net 4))
 (segment (start 175.2551 97.5741) (end 189.1879 97.5741) (width 0.25) (layer F.Cu) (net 4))
 (segment (start 189.1879 97.5741) (end 189.1879 100.9169) (width 0.25) (layer F.Cu) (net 4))
 (segment (start 189.1879 100.9169) (end 191.011 102.74) (width 0.25) (layer F.Cu) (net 4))
 (segment (start 172.9521 101.6211) (end 174.071 102.74) (width 0.25) (layer B.Cu) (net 4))
 (segment (start 165.76 100.3588) (end 171.6898 100.3588) (width 0.25) (layer B.Cu) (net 4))
 (segment (start 171.6898 100.3588) (end 172.9521 101.6211) (width 0.25) (layer B.Cu) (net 4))
 (segment (start 174.071 96.39) (end 174.4607 96.7797) (width 0.25) (layer B.Cu) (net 4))
 (segment (start 174.4607 96.7797) (end 174.4607 100.1125) (width 0.25) (layer B.Cu) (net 4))
 (segment (start 174.4607 100.1125) (end 172.9521 101.6211) (width 0.25) (layer B.Cu) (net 4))
 (segment (start 165.76 100.3588) (end 165.76 100.9465) (width 0.25) (layer B.Cu) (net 4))
 (segment (start 165.76 99.7712) (end 165.76 100.3588) (width 0.25) (layer B.Cu) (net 4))
 (segment (start 157.5679 102.3131) (end 157.141 102.74) (width 0.25) (layer B.Cu) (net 4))
 (segment (start 157.141 96.39) (end 157.5679 96.8169) (width 0.25) (layer B.Cu) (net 4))
 (segment (start 157.5679 96.8169) (end 157.5679 102.3131) (width 0.25) (layer B.Cu) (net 4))
 (segment (start 157.5679 102.3131) (end 159.1845 103.9297) (width 0.25) (layer B.Cu) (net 4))
 (segment (start 159.1845 103.9297) (end 162.0691 103.9297) (width 0.25) (layer B.Cu) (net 4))
 (segment (start 162.0691 103.9297) (end 165.0523 100.9465) (width 0.25) (layer B.Cu) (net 4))
 (segment (start 165.0523 100.9465) (end 165.76 100.9465) (width 0.25) (layer B.Cu) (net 4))
 (segment (start 89.7949 100.8182) (end 89.7949 102.3561) (width 0.25) (layer F.Cu) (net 5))
 (segment (start 89.7949 102.3561) (end 89.411 102.74) (width 0.25) (layer F.Cu) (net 5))
 (segment (start 89.411 96.39) (end 89.7949 96.7739) (width 0.25) (layer F.Cu) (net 5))
 (segment (start 89.7949 96.7739) (end 89.7949 100.8182) (width 0.25) (layer F.Cu) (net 5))
 (segment (start 89.7949 100.8182) (end 104.5186 100.8182) (width 0.25) (layer F.Cu) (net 5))
 (segment (start 104.5186 100.8182) (end 104.5186 99.1787) (width 0.25) (layer F.Cu) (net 5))
 (segment (start 104.5186 99.1787) (end 106.1131 97.5842) (width 0.25) (layer F.Cu) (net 5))
 (segment (start 106.1131 97.5842) (end 106.341 97.5842) (width 0.25) (layer F.Cu) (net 5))
 (segment (start 106.341 102.74) (end 104.5186 100.9176) (width 0.25) (layer F.Cu) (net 5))
 (segment (start 104.5186 100.9176) (end 104.5186 100.8182) (width 0.25) (layer F.Cu) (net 5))
 (segment (start 106.341 97.5842) (end 123.271 97.5842) (width 0.25) (layer F.Cu) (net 5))
 (segment (start 106.341 97.5842) (end 106.341 96.39) (width 0.25) (layer F.Cu) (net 5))
 (segment (start 123.271 97.5842) (end 128.2 97.5842) (width 0.25) (layer F.Cu) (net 5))
 (segment (start 128.2 97.5842) (end 130.084 95.7002) (width 0.25) (layer F.Cu) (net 5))
 (segment (start 130.084 95.7002) (end 133.1534 95.7002) (width 0.25) (layer F.Cu) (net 5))
 (segment (start 133.1534 95.7002) (end 134.199 96.7458) (width 0.25) (layer F.Cu) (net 5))
 (segment (start 134.199 96.7458) (end 138.1009 96.7458) (width 0.25) (layer F.Cu) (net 5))
 (segment (start 138.1009 96.7458) (end 138.9205 97.5654) (width 0.25) (layer F.Cu) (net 5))
 (segment (start 138.9205 97.5654) (end 164.2505 97.5654) (width 0.25) (layer F.Cu) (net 5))
 (segment (start 164.2505 97.5654) (end 164.5847 97.2312) (width 0.25) (layer F.Cu) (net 5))
 (segment (start 123.271 96.39) (end 123.271 97.5842) (width 0.25) (layer F.Cu) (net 5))
 (segment (start 165.76 97.2312) (end 164.5847 97.2312) (width 0.25) (layer F.Cu) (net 5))
 (segment (start 123.271 102.74) (end 123.6947 102.3163) (width 0.25) (layer B.Cu) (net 5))
 (segment (start 123.6947 102.3163) (end 123.6947 96.8137) (width 0.25) (layer B.Cu) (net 5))
 (segment (start 123.6947 96.8137) (end 123.271 96.39) (width 0.25) (layer B.Cu) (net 5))
 (segment (start 140.211 96.39) (end 141.4252 95.1758) (width 0.25) (layer F.Cu) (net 6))
 (segment (start 141.4252 95.1758) (end 145.1041 95.1758) (width 0.25) (layer F.Cu) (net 6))
 (segment (start 145.1041 95.1758) (end 146.8674 96.9391) (width 0.25) (layer F.Cu) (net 6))
 (segment (start 146.8674 96.9391) (end 153.3943 96.9391) (width 0.25) (layer F.Cu) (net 6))
 (segment (start 153.3943 96.9391) (end 155.6422 94.6912) (width 0.25) (layer F.Cu) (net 6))
 (segment (start 155.6422 94.6912) (end 165.76 94.6912) (width 0.25) (layer F.Cu) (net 6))
 (segment (start 140.211 96.39) (end 140.5949 96.7739) (width 0.25) (layer B.Cu) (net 6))
 (segment (start 140.5949 96.7739) (end 140.5949 102.3561) (width 0.25) (layer B.Cu) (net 6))
 (segment (start 140.5949 102.3561) (end 140.211 102.74) (width 0.25) (layer B.Cu) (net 6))
 (segment (start 179.151 99.565) (end 190.26 99.565) (width 0.25) (layer B.Cu) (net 19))
 (segment (start 190.26 99.565) (end 190.3 99.605) (width 0.25) (layer B.Cu) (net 19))
 (segment (start 162.221 99.565) (end 163.2183 98.5677) (width 0.25) (layer B.Cu) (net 20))
 (segment (start 163.2183 98.5677) (end 172.3227 98.5677) (width 0.25) (layer B.Cu) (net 20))
 (segment (start 172.3227 98.5677) (end 173.36 99.605) (width 0.25) (layer B.Cu) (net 20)))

